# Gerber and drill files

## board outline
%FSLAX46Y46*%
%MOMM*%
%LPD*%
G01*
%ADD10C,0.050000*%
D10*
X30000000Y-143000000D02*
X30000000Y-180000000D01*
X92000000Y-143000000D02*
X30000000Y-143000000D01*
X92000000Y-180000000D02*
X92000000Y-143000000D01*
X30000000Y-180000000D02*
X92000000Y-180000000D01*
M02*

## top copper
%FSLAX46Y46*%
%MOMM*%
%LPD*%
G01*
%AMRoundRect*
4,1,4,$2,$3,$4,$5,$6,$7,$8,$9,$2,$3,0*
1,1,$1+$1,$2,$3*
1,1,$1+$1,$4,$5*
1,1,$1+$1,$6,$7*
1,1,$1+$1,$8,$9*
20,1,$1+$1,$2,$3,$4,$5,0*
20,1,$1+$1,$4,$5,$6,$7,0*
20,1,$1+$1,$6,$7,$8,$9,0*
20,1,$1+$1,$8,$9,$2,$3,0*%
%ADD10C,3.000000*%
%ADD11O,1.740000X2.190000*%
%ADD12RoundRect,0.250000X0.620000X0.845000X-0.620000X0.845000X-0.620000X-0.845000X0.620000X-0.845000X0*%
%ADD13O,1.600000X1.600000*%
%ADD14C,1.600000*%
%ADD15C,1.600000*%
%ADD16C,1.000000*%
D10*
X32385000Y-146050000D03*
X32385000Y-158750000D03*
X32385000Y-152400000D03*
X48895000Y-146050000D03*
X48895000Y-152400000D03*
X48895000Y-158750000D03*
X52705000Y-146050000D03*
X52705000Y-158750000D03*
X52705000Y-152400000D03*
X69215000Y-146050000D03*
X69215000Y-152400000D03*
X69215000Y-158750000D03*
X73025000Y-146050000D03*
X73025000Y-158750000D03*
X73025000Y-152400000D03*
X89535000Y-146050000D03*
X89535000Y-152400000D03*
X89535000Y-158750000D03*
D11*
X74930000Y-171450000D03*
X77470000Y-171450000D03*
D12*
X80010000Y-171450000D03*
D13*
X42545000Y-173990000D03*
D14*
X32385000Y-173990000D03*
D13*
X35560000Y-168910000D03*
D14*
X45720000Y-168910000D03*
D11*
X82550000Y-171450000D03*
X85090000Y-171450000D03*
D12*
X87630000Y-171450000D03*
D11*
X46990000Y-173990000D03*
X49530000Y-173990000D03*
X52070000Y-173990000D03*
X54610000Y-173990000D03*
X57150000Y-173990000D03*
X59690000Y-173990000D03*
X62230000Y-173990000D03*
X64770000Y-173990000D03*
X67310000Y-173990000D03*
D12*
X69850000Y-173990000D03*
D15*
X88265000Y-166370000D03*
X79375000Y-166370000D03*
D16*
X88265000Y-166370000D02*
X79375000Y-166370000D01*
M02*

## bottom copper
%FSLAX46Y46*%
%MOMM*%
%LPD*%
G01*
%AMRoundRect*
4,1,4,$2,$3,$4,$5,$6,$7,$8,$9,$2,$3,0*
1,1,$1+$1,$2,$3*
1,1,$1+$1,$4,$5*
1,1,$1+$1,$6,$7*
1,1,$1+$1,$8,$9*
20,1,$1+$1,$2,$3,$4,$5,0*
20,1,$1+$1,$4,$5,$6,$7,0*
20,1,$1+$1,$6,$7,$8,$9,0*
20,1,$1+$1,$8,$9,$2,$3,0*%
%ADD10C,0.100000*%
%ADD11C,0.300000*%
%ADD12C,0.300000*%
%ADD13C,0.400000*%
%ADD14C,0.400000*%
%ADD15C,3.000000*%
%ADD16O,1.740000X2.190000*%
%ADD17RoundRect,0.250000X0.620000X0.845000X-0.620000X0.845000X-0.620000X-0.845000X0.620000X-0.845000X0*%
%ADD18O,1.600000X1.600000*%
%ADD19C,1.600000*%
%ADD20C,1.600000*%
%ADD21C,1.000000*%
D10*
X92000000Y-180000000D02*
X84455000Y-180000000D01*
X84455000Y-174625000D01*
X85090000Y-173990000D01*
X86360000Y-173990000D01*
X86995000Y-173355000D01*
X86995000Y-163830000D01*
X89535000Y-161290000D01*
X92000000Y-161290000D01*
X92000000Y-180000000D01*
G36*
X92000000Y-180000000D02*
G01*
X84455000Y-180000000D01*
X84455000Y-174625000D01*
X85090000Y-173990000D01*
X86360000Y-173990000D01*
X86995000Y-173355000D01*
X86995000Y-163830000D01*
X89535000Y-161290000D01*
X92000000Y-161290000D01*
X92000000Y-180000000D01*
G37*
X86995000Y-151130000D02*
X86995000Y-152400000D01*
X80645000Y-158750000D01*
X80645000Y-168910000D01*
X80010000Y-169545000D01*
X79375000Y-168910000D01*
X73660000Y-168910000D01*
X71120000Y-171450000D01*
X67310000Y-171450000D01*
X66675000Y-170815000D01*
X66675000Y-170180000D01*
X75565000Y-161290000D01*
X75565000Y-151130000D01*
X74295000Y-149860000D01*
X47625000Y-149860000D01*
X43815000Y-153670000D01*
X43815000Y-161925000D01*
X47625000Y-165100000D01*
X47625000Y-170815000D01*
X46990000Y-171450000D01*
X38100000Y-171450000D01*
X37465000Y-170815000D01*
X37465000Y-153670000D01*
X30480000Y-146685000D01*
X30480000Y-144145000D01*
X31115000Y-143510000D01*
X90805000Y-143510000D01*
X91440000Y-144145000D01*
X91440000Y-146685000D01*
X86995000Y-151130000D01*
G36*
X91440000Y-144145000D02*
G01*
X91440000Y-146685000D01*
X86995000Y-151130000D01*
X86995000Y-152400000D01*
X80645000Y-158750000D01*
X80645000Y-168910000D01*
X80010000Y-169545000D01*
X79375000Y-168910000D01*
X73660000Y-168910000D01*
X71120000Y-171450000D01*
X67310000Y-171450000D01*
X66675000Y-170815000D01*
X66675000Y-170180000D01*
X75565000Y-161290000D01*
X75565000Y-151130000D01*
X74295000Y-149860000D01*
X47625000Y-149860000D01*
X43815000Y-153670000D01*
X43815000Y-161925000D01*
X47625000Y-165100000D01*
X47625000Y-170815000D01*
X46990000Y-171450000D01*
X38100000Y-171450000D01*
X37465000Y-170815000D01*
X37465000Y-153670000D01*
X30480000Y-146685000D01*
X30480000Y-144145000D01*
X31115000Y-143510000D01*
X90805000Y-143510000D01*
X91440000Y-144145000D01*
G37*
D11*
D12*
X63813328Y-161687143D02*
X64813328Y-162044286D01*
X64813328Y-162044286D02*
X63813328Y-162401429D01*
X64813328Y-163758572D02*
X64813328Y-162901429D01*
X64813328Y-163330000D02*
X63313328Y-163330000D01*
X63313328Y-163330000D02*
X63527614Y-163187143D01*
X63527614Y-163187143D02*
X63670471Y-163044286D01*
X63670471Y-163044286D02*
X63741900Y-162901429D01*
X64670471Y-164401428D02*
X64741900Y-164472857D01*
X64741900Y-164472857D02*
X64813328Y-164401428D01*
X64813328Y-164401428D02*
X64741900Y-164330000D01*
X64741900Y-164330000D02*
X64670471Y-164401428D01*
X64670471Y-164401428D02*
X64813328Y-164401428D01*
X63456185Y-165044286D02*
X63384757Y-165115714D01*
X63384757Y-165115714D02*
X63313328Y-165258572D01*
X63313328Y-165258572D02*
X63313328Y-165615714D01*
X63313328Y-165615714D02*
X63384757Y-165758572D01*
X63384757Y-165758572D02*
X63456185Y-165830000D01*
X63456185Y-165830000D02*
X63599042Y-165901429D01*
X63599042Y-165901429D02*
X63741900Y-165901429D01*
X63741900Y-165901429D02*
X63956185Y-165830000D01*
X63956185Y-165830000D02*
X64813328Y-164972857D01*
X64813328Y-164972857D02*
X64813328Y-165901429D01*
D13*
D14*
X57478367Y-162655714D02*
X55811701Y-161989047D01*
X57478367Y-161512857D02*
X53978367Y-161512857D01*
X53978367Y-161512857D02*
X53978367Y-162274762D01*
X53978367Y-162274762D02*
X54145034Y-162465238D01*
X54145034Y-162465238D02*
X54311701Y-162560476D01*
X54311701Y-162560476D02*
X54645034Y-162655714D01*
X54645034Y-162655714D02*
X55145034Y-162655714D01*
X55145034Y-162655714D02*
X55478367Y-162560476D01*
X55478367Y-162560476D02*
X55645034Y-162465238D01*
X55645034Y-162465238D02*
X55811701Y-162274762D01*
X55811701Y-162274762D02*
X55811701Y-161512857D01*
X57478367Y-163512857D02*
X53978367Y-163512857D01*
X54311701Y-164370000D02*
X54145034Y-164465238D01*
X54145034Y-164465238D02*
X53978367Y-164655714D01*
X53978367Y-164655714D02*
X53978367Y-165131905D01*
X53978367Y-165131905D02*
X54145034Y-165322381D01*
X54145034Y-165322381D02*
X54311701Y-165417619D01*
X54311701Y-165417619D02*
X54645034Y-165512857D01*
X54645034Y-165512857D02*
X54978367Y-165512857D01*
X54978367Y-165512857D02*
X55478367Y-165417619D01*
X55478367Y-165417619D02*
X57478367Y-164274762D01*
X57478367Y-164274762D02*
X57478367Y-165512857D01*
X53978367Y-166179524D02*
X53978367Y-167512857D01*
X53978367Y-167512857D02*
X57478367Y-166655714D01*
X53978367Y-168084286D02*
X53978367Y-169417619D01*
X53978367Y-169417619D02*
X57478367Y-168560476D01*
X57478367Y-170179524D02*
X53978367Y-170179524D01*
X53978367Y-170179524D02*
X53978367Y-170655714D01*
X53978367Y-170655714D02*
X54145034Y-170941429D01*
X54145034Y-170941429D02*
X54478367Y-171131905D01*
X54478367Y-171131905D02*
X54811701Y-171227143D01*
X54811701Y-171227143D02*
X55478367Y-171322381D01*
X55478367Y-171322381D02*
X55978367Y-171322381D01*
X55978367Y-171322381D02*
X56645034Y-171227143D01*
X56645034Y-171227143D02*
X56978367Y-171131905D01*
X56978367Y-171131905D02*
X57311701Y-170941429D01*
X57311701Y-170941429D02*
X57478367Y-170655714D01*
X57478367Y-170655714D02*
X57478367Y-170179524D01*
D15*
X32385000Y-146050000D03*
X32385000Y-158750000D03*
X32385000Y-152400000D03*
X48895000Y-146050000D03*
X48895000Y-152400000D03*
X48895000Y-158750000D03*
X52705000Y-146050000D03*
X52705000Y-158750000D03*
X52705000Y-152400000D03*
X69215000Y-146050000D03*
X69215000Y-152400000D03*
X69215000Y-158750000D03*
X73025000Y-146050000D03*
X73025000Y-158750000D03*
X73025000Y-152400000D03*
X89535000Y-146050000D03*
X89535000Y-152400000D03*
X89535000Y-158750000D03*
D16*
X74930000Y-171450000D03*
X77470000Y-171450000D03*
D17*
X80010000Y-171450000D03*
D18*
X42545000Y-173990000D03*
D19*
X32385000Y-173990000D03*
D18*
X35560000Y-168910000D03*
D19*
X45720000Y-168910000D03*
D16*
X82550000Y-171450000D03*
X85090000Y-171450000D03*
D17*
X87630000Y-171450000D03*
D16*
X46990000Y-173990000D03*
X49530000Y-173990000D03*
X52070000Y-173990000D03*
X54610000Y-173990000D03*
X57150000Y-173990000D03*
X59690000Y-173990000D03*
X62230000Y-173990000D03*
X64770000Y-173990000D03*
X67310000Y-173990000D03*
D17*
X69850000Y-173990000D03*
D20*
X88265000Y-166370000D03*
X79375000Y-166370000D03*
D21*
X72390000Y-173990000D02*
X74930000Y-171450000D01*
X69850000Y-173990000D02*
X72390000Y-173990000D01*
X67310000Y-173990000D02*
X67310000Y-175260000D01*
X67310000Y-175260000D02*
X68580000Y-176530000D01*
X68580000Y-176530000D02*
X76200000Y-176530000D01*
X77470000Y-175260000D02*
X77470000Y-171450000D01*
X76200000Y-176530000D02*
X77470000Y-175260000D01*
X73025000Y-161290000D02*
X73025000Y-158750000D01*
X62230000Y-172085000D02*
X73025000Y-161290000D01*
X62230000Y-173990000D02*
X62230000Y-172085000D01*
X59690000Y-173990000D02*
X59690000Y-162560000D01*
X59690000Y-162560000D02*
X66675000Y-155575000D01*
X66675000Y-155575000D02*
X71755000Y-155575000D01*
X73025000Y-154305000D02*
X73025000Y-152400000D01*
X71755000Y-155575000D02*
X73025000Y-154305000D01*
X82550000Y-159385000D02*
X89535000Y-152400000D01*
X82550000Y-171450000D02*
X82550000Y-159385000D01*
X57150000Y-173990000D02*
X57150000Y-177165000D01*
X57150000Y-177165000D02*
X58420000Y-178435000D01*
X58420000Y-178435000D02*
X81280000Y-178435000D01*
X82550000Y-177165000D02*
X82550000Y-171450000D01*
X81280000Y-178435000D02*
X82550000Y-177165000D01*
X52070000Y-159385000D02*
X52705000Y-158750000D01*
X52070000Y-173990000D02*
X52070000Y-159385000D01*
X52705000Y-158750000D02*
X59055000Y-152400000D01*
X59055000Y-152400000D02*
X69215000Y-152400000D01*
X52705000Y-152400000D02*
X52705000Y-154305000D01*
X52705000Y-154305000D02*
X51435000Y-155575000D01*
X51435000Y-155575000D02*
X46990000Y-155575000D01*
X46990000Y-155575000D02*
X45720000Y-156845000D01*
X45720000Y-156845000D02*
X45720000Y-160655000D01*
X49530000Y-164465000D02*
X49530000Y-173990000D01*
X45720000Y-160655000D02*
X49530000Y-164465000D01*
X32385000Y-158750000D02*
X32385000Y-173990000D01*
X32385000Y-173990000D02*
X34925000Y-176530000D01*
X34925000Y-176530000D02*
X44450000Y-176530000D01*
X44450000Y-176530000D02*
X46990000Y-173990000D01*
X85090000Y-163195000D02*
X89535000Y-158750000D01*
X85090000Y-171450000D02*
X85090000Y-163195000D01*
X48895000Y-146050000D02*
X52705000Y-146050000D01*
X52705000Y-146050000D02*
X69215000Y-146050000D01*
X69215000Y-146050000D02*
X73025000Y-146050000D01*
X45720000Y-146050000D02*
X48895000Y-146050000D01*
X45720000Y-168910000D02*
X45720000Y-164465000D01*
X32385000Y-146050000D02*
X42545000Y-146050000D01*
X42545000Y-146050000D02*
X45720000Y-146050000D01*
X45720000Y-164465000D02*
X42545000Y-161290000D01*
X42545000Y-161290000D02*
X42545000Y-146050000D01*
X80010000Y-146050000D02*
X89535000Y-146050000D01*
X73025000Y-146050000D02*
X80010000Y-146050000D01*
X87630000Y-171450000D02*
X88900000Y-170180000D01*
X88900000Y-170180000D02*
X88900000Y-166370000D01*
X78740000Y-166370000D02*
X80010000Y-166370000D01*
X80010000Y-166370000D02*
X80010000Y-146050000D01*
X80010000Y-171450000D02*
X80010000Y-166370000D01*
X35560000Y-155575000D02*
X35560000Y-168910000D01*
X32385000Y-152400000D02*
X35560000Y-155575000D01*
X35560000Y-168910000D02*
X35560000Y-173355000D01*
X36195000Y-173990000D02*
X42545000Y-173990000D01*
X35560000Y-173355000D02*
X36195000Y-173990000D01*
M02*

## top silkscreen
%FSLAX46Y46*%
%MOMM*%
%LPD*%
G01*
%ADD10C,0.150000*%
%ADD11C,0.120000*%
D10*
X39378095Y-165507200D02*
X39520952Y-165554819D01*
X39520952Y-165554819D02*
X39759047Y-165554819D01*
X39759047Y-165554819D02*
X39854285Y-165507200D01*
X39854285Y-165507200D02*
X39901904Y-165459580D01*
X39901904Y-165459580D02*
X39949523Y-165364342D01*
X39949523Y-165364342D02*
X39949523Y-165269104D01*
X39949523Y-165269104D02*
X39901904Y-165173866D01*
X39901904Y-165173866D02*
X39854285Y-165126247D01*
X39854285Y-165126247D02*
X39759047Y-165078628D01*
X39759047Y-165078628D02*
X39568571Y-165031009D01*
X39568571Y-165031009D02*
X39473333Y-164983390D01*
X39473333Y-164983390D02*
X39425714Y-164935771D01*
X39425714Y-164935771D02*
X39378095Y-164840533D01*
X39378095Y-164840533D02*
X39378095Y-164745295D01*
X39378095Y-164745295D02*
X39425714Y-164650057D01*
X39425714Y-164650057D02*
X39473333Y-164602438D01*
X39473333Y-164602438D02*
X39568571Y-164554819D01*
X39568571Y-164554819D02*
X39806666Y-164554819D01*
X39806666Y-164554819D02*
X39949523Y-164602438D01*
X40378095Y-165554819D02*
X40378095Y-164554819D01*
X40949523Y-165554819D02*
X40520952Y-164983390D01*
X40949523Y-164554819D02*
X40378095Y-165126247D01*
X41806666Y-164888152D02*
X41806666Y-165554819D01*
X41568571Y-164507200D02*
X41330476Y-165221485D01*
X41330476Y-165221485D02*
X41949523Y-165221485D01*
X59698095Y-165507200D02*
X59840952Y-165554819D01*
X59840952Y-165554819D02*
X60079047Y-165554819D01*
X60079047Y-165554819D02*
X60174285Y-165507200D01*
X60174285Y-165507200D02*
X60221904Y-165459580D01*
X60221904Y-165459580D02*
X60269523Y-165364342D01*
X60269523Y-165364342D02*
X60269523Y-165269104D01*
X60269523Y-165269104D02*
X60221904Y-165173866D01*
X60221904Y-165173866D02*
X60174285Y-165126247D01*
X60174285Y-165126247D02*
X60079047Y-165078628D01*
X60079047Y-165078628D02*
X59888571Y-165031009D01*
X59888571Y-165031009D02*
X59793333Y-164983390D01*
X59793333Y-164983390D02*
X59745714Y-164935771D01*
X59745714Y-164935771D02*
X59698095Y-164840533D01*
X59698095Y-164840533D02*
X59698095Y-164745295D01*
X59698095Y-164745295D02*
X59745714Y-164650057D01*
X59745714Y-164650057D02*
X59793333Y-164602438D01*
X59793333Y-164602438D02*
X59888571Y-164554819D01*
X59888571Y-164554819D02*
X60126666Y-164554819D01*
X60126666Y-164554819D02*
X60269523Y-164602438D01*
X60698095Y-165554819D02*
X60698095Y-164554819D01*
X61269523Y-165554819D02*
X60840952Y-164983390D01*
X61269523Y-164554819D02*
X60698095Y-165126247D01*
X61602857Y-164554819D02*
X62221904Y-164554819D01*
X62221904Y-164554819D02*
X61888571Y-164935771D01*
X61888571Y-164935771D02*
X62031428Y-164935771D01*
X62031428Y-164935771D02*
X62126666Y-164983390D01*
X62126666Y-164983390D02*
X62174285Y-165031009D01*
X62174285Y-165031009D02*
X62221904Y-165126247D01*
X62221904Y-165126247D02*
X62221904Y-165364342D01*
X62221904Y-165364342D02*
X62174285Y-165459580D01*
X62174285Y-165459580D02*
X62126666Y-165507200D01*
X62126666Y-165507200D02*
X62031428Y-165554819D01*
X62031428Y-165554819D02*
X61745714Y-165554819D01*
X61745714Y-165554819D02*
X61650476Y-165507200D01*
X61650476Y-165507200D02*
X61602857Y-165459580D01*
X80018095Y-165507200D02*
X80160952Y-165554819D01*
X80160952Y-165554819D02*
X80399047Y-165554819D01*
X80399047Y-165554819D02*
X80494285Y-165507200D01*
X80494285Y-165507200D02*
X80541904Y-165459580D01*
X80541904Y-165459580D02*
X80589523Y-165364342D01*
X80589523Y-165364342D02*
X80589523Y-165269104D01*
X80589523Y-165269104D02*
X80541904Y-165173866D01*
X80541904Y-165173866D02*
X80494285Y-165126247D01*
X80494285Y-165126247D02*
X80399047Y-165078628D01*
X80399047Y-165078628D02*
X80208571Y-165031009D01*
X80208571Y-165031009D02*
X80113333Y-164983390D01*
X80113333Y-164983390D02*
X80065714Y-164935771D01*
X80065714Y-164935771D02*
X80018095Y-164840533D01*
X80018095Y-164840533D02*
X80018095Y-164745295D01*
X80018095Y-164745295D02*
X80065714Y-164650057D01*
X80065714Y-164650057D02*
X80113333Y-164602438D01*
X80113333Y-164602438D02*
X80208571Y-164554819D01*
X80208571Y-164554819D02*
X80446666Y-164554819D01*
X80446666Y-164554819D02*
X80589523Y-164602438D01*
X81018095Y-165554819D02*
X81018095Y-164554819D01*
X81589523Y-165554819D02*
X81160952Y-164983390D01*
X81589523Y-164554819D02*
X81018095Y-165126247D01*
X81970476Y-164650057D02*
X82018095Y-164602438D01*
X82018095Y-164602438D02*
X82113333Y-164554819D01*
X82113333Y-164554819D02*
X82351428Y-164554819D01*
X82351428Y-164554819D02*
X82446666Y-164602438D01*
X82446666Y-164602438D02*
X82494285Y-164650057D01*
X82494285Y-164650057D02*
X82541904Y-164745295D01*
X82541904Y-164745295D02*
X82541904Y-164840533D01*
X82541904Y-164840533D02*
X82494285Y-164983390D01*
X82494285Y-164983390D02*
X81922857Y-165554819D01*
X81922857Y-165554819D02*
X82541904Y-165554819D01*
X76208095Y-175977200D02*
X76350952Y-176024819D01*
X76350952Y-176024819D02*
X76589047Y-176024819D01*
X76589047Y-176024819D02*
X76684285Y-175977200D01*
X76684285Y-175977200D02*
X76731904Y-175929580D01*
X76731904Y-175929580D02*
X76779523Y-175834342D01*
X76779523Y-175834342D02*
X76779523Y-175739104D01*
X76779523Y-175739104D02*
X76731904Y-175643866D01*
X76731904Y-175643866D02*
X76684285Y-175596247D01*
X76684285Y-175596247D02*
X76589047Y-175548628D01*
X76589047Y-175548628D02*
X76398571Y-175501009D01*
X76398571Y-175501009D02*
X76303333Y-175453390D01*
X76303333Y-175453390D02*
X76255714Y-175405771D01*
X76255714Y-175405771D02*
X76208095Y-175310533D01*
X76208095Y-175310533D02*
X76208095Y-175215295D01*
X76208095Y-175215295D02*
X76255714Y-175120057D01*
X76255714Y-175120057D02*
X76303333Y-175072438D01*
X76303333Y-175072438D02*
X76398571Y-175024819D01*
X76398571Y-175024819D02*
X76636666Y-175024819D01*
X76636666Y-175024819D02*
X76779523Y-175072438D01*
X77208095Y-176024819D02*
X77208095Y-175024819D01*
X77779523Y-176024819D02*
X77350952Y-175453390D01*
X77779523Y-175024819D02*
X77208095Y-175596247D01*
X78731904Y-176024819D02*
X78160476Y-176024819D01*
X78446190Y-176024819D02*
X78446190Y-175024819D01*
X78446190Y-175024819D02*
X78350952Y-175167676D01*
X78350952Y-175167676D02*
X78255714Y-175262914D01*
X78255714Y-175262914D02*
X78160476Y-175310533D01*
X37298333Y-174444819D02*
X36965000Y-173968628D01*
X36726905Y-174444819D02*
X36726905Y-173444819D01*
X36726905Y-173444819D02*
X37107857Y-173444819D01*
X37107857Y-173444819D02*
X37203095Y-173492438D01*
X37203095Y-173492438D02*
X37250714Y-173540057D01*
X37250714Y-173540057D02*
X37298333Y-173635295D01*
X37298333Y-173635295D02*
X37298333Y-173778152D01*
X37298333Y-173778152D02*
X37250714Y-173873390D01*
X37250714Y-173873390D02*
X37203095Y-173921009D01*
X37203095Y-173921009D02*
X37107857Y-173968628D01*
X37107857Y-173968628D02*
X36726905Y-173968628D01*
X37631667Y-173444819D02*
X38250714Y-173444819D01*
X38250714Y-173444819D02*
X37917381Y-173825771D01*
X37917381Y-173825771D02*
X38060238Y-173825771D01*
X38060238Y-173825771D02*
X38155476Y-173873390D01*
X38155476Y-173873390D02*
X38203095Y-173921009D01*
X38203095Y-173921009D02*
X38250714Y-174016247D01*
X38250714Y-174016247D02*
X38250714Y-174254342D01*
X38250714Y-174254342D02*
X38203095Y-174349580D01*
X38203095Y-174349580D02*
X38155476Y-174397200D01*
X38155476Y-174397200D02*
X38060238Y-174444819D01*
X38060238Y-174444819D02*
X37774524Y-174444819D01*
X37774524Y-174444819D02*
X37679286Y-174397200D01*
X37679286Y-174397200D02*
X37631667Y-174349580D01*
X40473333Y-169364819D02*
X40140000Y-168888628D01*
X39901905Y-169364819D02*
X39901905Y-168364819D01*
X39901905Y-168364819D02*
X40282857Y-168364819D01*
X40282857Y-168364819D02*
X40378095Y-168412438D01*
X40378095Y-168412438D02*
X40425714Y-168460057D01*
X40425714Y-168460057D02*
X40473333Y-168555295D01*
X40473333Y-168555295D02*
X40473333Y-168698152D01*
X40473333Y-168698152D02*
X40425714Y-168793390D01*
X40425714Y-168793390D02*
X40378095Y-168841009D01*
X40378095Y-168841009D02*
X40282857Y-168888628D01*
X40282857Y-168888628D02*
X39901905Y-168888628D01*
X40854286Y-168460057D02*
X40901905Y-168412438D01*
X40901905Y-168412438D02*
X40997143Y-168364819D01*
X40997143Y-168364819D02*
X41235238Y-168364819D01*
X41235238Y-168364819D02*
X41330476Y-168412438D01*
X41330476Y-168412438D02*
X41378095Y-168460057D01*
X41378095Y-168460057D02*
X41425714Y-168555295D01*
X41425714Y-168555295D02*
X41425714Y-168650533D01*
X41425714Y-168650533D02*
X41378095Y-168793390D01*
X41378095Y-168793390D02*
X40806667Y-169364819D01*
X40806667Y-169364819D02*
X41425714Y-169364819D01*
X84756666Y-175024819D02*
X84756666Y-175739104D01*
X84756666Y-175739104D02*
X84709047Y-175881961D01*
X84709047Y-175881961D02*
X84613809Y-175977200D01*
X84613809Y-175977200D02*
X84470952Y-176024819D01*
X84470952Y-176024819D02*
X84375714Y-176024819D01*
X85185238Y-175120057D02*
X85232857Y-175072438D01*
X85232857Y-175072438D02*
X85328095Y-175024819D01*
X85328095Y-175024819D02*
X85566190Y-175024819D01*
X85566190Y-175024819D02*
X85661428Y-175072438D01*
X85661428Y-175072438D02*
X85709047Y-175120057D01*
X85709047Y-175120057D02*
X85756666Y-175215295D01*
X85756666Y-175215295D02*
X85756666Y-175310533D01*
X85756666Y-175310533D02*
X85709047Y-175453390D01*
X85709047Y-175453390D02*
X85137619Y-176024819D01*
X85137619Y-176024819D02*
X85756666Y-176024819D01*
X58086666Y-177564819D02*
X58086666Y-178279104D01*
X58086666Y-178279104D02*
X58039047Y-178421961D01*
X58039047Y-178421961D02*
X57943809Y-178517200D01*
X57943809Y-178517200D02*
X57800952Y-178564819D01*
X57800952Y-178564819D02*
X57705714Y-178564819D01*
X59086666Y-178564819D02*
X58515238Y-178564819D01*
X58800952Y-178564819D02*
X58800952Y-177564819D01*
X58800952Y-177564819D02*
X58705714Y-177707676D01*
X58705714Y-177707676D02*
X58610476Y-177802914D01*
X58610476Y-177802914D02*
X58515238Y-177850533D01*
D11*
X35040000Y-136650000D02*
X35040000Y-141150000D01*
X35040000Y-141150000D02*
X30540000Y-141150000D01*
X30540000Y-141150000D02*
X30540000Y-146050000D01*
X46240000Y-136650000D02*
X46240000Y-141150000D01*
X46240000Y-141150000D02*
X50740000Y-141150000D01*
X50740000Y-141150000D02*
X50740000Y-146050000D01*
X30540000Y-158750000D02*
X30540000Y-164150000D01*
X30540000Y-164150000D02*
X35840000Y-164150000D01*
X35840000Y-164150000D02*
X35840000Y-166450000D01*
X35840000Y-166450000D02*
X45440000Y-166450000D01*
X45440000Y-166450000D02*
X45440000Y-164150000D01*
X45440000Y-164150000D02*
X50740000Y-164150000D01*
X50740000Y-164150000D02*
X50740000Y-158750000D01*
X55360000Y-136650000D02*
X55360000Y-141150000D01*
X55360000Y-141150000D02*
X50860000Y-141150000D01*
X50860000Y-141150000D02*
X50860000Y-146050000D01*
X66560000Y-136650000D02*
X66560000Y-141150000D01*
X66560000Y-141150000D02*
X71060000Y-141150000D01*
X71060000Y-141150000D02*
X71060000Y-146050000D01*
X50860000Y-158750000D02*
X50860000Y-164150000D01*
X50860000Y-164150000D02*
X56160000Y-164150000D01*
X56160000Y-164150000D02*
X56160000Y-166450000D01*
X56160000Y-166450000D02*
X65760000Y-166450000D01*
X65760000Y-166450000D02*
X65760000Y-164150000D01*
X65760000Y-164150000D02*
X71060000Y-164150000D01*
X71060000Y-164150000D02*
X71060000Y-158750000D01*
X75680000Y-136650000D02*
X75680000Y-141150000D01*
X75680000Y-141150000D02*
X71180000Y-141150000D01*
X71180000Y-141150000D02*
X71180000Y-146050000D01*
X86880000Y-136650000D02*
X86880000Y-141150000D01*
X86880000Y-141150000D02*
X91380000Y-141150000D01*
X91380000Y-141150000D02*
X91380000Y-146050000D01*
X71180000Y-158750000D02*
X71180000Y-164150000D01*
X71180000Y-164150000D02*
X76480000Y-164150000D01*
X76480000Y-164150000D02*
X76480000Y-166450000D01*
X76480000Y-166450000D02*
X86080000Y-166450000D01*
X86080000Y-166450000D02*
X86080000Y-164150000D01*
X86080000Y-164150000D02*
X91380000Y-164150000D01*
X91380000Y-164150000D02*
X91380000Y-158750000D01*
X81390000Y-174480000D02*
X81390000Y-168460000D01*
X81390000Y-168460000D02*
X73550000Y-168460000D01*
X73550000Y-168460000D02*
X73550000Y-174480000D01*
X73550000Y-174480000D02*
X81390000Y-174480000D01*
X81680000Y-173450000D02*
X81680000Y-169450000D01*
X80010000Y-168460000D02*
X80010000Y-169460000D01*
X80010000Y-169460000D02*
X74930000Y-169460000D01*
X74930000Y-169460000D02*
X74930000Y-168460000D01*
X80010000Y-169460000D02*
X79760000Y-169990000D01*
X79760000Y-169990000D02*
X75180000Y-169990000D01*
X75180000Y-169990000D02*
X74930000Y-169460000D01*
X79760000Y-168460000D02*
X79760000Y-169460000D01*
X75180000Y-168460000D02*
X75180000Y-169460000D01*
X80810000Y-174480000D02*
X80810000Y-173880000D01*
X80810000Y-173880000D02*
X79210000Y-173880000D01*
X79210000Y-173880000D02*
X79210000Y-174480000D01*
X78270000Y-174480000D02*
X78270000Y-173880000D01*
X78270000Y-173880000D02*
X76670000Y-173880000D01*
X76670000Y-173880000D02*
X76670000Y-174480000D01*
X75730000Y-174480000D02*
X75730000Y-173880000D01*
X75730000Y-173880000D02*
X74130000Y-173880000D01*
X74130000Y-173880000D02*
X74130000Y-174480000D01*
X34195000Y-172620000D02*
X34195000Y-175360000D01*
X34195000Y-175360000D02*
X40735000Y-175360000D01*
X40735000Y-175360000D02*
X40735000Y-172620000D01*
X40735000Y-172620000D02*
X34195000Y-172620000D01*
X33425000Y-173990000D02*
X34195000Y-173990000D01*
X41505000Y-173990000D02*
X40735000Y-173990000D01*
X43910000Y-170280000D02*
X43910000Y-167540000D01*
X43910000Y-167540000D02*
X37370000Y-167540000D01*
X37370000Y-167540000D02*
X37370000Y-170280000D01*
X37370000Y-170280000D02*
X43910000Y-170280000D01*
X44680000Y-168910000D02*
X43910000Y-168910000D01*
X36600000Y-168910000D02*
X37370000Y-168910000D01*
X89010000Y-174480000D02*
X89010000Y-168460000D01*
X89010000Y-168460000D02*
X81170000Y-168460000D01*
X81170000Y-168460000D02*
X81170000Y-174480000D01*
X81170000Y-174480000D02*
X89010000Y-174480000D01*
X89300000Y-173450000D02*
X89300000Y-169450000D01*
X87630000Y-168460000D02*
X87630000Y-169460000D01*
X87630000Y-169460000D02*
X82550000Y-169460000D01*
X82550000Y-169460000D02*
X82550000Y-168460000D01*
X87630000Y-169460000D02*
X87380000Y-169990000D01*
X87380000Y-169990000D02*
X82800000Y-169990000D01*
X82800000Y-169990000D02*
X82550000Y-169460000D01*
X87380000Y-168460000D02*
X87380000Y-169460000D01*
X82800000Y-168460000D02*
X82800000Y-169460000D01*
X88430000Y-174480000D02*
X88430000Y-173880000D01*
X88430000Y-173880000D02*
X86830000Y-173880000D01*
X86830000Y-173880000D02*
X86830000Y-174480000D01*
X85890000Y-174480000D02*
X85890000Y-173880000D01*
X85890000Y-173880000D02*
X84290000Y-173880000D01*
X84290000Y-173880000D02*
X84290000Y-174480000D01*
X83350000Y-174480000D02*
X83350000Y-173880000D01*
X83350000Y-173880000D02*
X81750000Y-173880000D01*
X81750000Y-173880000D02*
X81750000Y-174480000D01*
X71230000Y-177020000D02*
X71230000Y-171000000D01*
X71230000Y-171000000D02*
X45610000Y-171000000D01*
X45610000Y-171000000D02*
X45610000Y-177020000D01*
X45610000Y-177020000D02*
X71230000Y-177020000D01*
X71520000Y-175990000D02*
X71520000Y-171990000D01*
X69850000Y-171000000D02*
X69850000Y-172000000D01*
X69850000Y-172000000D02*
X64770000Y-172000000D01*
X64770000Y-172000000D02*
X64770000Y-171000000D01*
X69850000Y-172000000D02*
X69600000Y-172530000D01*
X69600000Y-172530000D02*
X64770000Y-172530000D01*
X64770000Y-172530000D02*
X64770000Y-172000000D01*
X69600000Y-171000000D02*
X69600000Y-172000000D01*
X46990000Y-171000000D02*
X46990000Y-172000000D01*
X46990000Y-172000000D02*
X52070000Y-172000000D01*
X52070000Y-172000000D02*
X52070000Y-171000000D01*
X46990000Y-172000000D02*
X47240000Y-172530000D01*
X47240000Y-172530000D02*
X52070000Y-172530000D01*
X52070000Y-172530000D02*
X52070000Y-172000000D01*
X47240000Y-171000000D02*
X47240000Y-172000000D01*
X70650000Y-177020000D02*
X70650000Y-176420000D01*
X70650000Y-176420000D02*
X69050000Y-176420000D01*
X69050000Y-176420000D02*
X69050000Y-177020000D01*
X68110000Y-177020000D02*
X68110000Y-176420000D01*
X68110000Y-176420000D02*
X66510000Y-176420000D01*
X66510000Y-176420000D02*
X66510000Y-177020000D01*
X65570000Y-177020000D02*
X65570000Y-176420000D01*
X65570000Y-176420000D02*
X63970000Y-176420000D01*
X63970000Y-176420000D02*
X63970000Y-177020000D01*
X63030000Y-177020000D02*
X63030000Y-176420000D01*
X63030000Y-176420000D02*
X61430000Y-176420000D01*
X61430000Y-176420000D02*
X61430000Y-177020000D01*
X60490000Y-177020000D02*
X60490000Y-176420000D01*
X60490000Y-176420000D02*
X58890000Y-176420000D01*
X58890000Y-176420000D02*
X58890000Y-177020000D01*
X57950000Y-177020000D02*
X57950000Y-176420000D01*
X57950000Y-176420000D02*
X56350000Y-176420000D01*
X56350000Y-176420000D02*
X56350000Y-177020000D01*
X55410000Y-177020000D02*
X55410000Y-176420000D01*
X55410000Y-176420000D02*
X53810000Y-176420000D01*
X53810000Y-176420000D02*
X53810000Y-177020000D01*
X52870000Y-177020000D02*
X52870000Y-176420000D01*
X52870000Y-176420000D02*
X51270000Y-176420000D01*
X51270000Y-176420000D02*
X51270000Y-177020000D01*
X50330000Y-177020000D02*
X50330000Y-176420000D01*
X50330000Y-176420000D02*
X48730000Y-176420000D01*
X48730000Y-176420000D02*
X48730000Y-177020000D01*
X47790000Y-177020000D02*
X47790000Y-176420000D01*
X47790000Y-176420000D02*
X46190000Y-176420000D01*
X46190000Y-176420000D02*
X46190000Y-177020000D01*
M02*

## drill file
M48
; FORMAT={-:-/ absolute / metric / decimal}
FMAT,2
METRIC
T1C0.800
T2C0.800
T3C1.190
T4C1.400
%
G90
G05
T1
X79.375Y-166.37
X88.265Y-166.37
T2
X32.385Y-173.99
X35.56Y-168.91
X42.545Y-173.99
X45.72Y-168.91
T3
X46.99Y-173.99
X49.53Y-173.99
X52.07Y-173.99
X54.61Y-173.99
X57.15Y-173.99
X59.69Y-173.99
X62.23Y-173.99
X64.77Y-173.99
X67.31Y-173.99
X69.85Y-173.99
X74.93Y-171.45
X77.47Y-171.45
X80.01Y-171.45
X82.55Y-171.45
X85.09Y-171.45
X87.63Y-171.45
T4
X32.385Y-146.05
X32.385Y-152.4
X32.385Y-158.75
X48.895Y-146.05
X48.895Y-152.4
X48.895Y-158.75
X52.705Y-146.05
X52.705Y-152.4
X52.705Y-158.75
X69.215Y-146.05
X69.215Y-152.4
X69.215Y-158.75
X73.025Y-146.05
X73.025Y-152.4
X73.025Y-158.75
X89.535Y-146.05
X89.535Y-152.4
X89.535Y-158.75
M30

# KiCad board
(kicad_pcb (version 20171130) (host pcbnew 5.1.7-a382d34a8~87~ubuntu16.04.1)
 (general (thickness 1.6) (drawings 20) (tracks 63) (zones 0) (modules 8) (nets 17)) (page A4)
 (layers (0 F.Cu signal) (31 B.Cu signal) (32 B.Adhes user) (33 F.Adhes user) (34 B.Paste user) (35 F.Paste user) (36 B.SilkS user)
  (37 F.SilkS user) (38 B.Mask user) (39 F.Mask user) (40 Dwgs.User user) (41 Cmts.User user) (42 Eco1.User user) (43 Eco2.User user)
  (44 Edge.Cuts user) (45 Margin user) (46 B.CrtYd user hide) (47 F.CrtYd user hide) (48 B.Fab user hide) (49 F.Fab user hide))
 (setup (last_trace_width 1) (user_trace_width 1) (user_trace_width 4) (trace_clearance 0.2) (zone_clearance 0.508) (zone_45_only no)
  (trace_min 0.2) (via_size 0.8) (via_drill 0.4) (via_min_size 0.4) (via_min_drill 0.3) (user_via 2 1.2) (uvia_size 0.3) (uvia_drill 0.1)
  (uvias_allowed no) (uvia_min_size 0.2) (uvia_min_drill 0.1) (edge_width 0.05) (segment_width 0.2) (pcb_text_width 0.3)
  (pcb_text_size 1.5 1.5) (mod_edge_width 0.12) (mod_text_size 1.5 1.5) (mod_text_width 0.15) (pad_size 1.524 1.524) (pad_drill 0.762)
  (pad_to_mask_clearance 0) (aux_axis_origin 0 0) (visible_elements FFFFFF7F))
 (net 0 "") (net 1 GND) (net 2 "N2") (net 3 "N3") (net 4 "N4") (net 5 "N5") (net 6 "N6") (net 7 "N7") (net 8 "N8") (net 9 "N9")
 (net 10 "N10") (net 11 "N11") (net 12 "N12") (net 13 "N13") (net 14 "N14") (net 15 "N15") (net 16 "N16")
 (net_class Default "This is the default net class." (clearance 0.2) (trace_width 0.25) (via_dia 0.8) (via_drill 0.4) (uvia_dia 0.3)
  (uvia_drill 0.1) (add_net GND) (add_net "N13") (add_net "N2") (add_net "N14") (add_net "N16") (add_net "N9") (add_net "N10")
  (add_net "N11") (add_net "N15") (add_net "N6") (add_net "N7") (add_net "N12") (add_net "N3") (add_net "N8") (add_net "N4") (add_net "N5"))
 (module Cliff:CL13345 (layer F.Cu) (at 40.64 146.05 90)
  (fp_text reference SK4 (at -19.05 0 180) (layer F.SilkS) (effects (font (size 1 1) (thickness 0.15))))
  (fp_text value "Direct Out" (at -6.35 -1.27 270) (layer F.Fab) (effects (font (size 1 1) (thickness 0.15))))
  (fp_line (start 9.4 -5.6) (end 4.9 -5.6) (layer F.SilkS) (width 0.12))
  (fp_line (start 4.9 -5.6) (end 4.9 -10.1) (layer F.SilkS) (width 0.12))
  (fp_line (start 4.9 -10.1) (end 0 -10.1) (layer F.SilkS) (width 0.12))
  (fp_line (start 9.4 5.6) (end 4.9 5.6) (layer F.SilkS) (width 0.12))
  (fp_line (start 4.9 5.6) (end 4.9 10.1) (layer F.SilkS) (width 0.12))
  (fp_line (start 4.9 10.1) (end 0 10.1) (layer F.SilkS) (width 0.12))
  (fp_line (start -12.7 -10.1) (end -18.1 -10.1) (layer F.SilkS) (width 0.12))
  (fp_line (start -18.1 -10.1) (end -18.1 -4.8) (layer F.SilkS) (width 0.12))
  (fp_line (start -18.1 -4.8) (end -20.4 -4.8) (layer F.SilkS) (width 0.12))
  (fp_line (start -20.4 -4.8) (end -20.4 4.8) (layer F.SilkS) (width 0.12))
  (fp_line (start -20.4 4.8) (end -18.1 4.8) (layer F.SilkS) (width 0.12))
  (fp_line (start -18.1 4.8) (end -18.1 10.1) (layer F.SilkS) (width 0.12))
  (fp_line (start -18.1 10.1) (end -12.7 10.1) (layer F.SilkS) (width 0.12))
  (pad S thru_hole circle (at 0 -8.255 180) (size 3 3) (drill 1.4) (layers *.Cu *.Mask) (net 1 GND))
  (pad T thru_hole circle (at -12.7 -8.255 180) (size 3 3) (drill 1.4) (layers *.Cu *.Mask) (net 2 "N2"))
  (pad R thru_hole circle (at -6.35 -8.255 180) (size 3 3) (drill 1.4) (layers *.Cu *.Mask) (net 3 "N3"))
  (pad SN thru_hole circle (at 0 8.255 180) (size 3 3) (drill 1.4) (layers *.Cu *.Mask) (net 1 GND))
  (pad RN thru_hole circle (at -6.35 8.255 180) (size 3 3) (drill 1.4) (layers *.Cu *.Mask) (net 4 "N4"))
  (pad TN thru_hole circle (at -12.7 8.255 180) (size 3 3) (drill 1.4) (layers *.Cu *.Mask) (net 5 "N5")))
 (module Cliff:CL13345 (layer F.Cu) (at 60.96 146.05 90)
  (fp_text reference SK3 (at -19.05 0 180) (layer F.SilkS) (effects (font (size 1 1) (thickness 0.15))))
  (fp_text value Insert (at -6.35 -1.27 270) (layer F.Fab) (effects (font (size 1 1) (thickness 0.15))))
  (fp_line (start 9.4 -5.6) (end 4.9 -5.6) (layer F.SilkS) (width 0.12))
  (fp_line (start 4.9 -5.6) (end 4.9 -10.1) (layer F.SilkS) (width 0.12))
  (fp_line (start 4.9 -10.1) (end 0 -10.1) (layer F.SilkS) (width 0.12))
  (fp_line (start 9.4 5.6) (end 4.9 5.6) (layer F.SilkS) (width 0.12))
  (fp_line (start 4.9 5.6) (end 4.9 10.1) (layer F.SilkS) (width 0.12))
  (fp_line (start 4.9 10.1) (end 0 10.1) (layer F.SilkS) (width 0.12))
  (fp_line (start -12.7 -10.1) (end -18.1 -10.1) (layer F.SilkS) (width 0.12))
  (fp_line (start -18.1 -10.1) (end -18.1 -4.8) (layer F.SilkS) (width 0.12))
  (fp_line (start -18.1 -4.8) (end -20.4 -4.8) (layer F.SilkS) (width 0.12))
  (fp_line (start -20.4 -4.8) (end -20.4 4.8) (layer F.SilkS) (width 0.12))
  (fp_line (start -20.4 4.8) (end -18.1 4.8) (layer F.SilkS) (width 0.12))
  (fp_line (start -18.1 4.8) (end -18.1 10.1) (layer F.SilkS) (width 0.12))
  (fp_line (start -18.1 10.1) (end -12.7 10.1) (layer F.SilkS) (width 0.12))
  (pad S thru_hole circle (at 0 -8.255 180) (size 3 3) (drill 1.4) (layers *.Cu *.Mask) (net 1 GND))
  (pad T thru_hole circle (at -12.7 -8.255 180) (size 3 3) (drill 1.4) (layers *.Cu *.Mask) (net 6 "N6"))
  (pad R thru_hole circle (at -6.35 -8.255 180) (size 3 3) (drill 1.4) (layers *.Cu *.Mask) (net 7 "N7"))
  (pad SN thru_hole circle (at 0 8.255 180) (size 3 3) (drill 1.4) (layers *.Cu *.Mask) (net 1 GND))
  (pad RN thru_hole circle (at -6.35 8.255 180) (size 3 3) (drill 1.4) (layers *.Cu *.Mask) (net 6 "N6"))
  (pad TN thru_hole circle (at -12.7 8.255 180) (size 3 3) (drill 1.4) (layers *.Cu *.Mask) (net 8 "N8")))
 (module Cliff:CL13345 (layer F.Cu) (at 81.28 146.05 90)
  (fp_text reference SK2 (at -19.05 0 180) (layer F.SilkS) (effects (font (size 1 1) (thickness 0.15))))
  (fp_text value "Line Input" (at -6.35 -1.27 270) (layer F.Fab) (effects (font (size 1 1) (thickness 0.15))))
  (fp_line (start 9.4 -5.6) (end 4.9 -5.6) (layer F.SilkS) (width 0.12))
  (fp_line (start 4.9 -5.6) (end 4.9 -10.1) (layer F.SilkS) (width 0.12))
  (fp_line (start 4.9 -10.1) (end 0 -10.1) (layer F.SilkS) (width 0.12))
  (fp_line (start 9.4 5.6) (end 4.9 5.6) (layer F.SilkS) (width 0.12))
  (fp_line (start 4.9 5.6) (end 4.9 10.1) (layer F.SilkS) (width 0.12))
  (fp_line (start 4.9 10.1) (end 0 10.1) (layer F.SilkS) (width 0.12))
  (fp_line (start -12.7 -10.1) (end -18.1 -10.1) (layer F.SilkS) (width 0.12))
  (fp_line (start -18.1 -10.1) (end -18.1 -4.8) (layer F.SilkS) (width 0.12))
  (fp_line (start -18.1 -4.8) (end -20.4 -4.8) (layer F.SilkS) (width 0.12))
  (fp_line (start -20.4 -4.8) (end -20.4 4.8) (layer F.SilkS) (width 0.12))
  (fp_line (start -20.4 4.8) (end -18.1 4.8) (layer F.SilkS) (width 0.12))
  (fp_line (start -18.1 4.8) (end -18.1 10.1) (layer F.SilkS) (width 0.12))
  (fp_line (start -18.1 10.1) (end -12.7 10.1) (layer F.SilkS) (width 0.12))
  (pad S thru_hole circle (at 0 -8.255 180) (size 3 3) (drill 1.4) (layers *.Cu *.Mask) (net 1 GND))
  (pad T thru_hole circle (at -12.7 -8.255 180) (size 3 3) (drill 1.4) (layers *.Cu *.Mask) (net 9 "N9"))
  (pad R thru_hole circle (at -6.35 -8.255 180) (size 3 3) (drill 1.4) (layers *.Cu *.Mask) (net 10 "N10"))
  (pad SN thru_hole circle (at 0 8.255 180) (size 3 3) (drill 1.4) (layers *.Cu *.Mask) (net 1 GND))
  (pad RN thru_hole circle (at -6.35 8.255 180) (size 3 3) (drill 1.4) (layers *.Cu *.Mask) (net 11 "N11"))
  (pad TN thru_hole circle (at -12.7 8.255 180) (size 3 3) (drill 1.4) (layers *.Cu *.Mask) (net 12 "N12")))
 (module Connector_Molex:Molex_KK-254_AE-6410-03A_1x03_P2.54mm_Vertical (layer F.Cu) (at 80.01 171.45 180)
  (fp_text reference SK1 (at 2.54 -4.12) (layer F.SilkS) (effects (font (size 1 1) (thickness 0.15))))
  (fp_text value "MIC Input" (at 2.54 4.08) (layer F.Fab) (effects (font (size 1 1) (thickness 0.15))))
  (fp_line (start -1.38 -3.03) (end -1.38 2.99) (layer F.SilkS) (width 0.12))
  (fp_line (start -1.38 2.99) (end 6.46 2.99) (layer F.SilkS) (width 0.12))
  (fp_line (start 6.46 2.99) (end 6.46 -3.03) (layer F.SilkS) (width 0.12))
  (fp_line (start 6.46 -3.03) (end -1.38 -3.03) (layer F.SilkS) (width 0.12))
  (fp_line (start -1.67 -2) (end -1.67 2) (layer F.SilkS) (width 0.12))
  (fp_line (start 0 2.99) (end 0 1.99) (layer F.SilkS) (width 0.12))
  (fp_line (start 0 1.99) (end 5.08 1.99) (layer F.SilkS) (width 0.12))
  (fp_line (start 5.08 1.99) (end 5.08 2.99) (layer F.SilkS) (width 0.12))
  (fp_line (start 0 1.99) (end 0.25 1.46) (layer F.SilkS) (width 0.12))
  (fp_line (start 0.25 1.46) (end 4.83 1.46) (layer F.SilkS) (width 0.12))
  (fp_line (start 4.83 1.46) (end 5.08 1.99) (layer F.SilkS) (width 0.12))
  (fp_line (start 0.25 2.99) (end 0.25 1.99) (layer F.SilkS) (width 0.12))
  (fp_line (start 4.83 2.99) (end 4.83 1.99) (layer F.SilkS) (width 0.12))
  (fp_line (start -0.8 -3.03) (end -0.8 -2.43) (layer F.SilkS) (width 0.12))
  (fp_line (start -0.8 -2.43) (end 0.8 -2.43) (layer F.SilkS) (width 0.12))
  (fp_line (start 0.8 -2.43) (end 0.8 -3.03) (layer F.SilkS) (width 0.12))
  (fp_line (start 1.74 -3.03) (end 1.74 -2.43) (layer F.SilkS) (width 0.12))
  (fp_line (start 1.74 -2.43) (end 3.34 -2.43) (layer F.SilkS) (width 0.12))
  (fp_line (start 3.34 -2.43) (end 3.34 -3.03) (layer F.SilkS) (width 0.12))
  (fp_line (start 4.28 -3.03) (end 4.28 -2.43) (layer F.SilkS) (width 0.12))
  (fp_line (start 4.28 -2.43) (end 5.88 -2.43) (layer F.SilkS) (width 0.12))
  (fp_line (start 5.88 -2.43) (end 5.88 -3.03) (layer F.SilkS) (width 0.12))
  (pad 3 thru_hole oval (at 5.08 0 180) (size 1.74 2.19) (drill 1.19) (layers *.Cu *.Mask) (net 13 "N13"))
  (pad 2 thru_hole oval (at 2.54 0 180) (size 1.74 2.19) (drill 1.19) (layers *.Cu *.Mask) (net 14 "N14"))
  (pad 1 thru_hole roundrect (at 0 0 180) (size 1.74 2.19) (drill 1.19) (layers *.Cu *.Mask) (roundrect_rratio 0.143678) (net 1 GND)))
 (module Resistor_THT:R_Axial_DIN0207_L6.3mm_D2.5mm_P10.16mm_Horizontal (layer F.Cu) (at 32.385 173.99)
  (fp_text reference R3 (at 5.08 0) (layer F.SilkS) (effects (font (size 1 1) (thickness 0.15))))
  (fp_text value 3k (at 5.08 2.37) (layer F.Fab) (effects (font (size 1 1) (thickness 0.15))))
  (fp_line (start 1.81 -1.37) (end 1.81 1.37) (layer F.SilkS) (width 0.12))
  (fp_line (start 1.81 1.37) (end 8.35 1.37) (layer F.SilkS) (width 0.12))
  (fp_line (start 8.35 1.37) (end 8.35 -1.37) (layer F.SilkS) (width 0.12))
  (fp_line (start 8.35 -1.37) (end 1.81 -1.37) (layer F.SilkS) (width 0.12))
  (fp_line (start 1.04 0) (end 1.81 0) (layer F.SilkS) (width 0.12))
  (fp_line (start 9.12 0) (end 8.35 0) (layer F.SilkS) (width 0.12))
  (pad 2 thru_hole oval (at 10.16 0) (size 1.6 1.6) (drill 0.8) (layers *.Cu *.Mask) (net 3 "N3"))
  (pad 1 thru_hole circle (at 0 0) (size 1.6 1.6) (drill 0.8) (layers *.Cu *.Mask) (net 2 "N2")))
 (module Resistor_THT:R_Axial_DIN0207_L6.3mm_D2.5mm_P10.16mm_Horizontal (layer F.Cu) (at 45.72 168.91 180)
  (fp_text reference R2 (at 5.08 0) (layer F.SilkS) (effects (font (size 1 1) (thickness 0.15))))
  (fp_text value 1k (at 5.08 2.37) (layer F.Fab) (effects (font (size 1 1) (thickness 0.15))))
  (fp_line (start 1.81 -1.37) (end 1.81 1.37) (layer F.SilkS) (width 0.12))
  (fp_line (start 1.81 1.37) (end 8.35 1.37) (layer F.SilkS) (width 0.12))
  (fp_line (start 8.35 1.37) (end 8.35 -1.37) (layer F.SilkS) (width 0.12))
  (fp_line (start 8.35 -1.37) (end 1.81 -1.37) (layer F.SilkS) (width 0.12))
  (fp_line (start 1.04 0) (end 1.81 0) (layer F.SilkS) (width 0.12))
  (fp_line (start 9.12 0) (end 8.35 0) (layer F.SilkS) (width 0.12))
  (pad 2 thru_hole oval (at 10.16 0 180) (size 1.6 1.6) (drill 0.8) (layers *.Cu *.Mask) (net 3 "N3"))
  (pad 1 thru_hole circle (at 0 0 180) (size 1.6 1.6) (drill 0.8) (layers *.Cu *.Mask) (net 1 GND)))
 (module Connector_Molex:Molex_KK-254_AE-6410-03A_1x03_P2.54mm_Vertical (layer F.Cu) (at 87.63 171.45 180)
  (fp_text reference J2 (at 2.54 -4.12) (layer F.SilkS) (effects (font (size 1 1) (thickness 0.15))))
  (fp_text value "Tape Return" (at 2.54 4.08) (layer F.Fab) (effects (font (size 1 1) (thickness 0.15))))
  (fp_line (start -1.38 -3.03) (end -1.38 2.99) (layer F.SilkS) (width 0.12))
  (fp_line (start -1.38 2.99) (end 6.46 2.99) (layer F.SilkS) (width 0.12))
  (fp_line (start 6.46 2.99) (end 6.46 -3.03) (layer F.SilkS) (width 0.12))
  (fp_line (start 6.46 -3.03) (end -1.38 -3.03) (layer F.SilkS) (width 0.12))
  (fp_line (start -1.67 -2) (end -1.67 2) (layer F.SilkS) (width 0.12))
  (fp_line (start 0 2.99) (end 0 1.99) (layer F.SilkS) (width 0.12))
  (fp_line (start 0 1.99) (end 5.08 1.99) (layer F.SilkS) (width 0.12))
  (fp_line (start 5.08 1.99) (end 5.08 2.99) (layer F.SilkS) (width 0.12))
  (fp_line (start 0 1.99) (end 0.25 1.46) (layer F.SilkS) (width 0.12))
  (fp_line (start 0.25 1.46) (end 4.83 1.46) (layer F.SilkS) (width 0.12))
  (fp_line (start 4.83 1.46) (end 5.08 1.99) (layer F.SilkS) (width 0.12))
  (fp_line (start 0.25 2.99) (end 0.25 1.99) (layer F.SilkS) (width 0.12))
  (fp_line (start 4.83 2.99) (end 4.83 1.99) (layer F.SilkS) (width 0.12))
  (fp_line (start -0.8 -3.03) (end -0.8 -2.43) (layer F.SilkS) (width 0.12))
  (fp_line (start -0.8 -2.43) (end 0.8 -2.43) (layer F.SilkS) (width 0.12))
  (fp_line (start 0.8 -2.43) (end 0.8 -3.03) (layer F.SilkS) (width 0.12))
  (fp_line (start 1.74 -3.03) (end 1.74 -2.43) (layer F.SilkS) (width 0.12))
  (fp_line (start 1.74 -2.43) (end 3.34 -2.43) (layer F.SilkS) (width 0.12))
  (fp_line (start 3.34 -2.43) (end 3.34 -3.03) (layer F.SilkS) (width 0.12))
  (fp_line (start 4.28 -3.03) (end 4.28 -2.43) (layer F.SilkS) (width 0.12))
  (fp_line (start 4.28 -2.43) (end 5.88 -2.43) (layer F.SilkS) (width 0.12))
  (fp_line (start 5.88 -2.43) (end 5.88 -3.03) (layer F.SilkS) (width 0.12))
  (pad 3 thru_hole oval (at 5.08 0 180) (size 1.74 2.19) (drill 1.19) (layers *.Cu *.Mask) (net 11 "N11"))
  (pad 2 thru_hole oval (at 2.54 0 180) (size 1.74 2.19) (drill 1.19) (layers *.Cu *.Mask) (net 12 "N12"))
  (pad 1 thru_hole roundrect (at 0 0 180) (size 1.74 2.19) (drill 1.19) (layers *.Cu *.Mask) (roundrect_rratio 0.143678) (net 1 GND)))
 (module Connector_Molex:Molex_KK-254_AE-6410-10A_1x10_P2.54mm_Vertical (layer F.Cu) (at 69.85 173.99 180)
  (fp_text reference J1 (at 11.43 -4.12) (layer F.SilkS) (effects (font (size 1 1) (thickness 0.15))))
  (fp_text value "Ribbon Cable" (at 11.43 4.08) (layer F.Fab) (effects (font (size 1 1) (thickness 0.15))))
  (fp_line (start -1.38 -3.03) (end -1.38 2.99) (layer F.SilkS) (width 0.12))
  (fp_line (start -1.38 2.99) (end 24.24 2.99) (layer F.SilkS) (width 0.12))
  (fp_line (start 24.24 2.99) (end 24.24 -3.03) (layer F.SilkS) (width 0.12))
  (fp_line (start 24.24 -3.03) (end -1.38 -3.03) (layer F.SilkS) (width 0.12))
  (fp_line (start -1.67 -2) (end -1.67 2) (layer F.SilkS) (width 0.12))
  (fp_line (start 0 2.99) (end 0 1.99) (layer F.SilkS) (width 0.12))
  (fp_line (start 0 1.99) (end 5.08 1.99) (layer F.SilkS) (width 0.12))
  (fp_line (start 5.08 1.99) (end 5.08 2.99) (layer F.SilkS) (width 0.12))
  (fp_line (start 0 1.99) (end 0.25 1.46) (layer F.SilkS) (width 0.12))
  (fp_line (start 0.25 1.46) (end 5.08 1.46) (layer F.SilkS) (width 0.12))
  (fp_line (start 5.08 1.46) (end 5.08 1.99) (layer F.SilkS) (width 0.12))
  (fp_line (start 0.25 2.99) (end 0.25 1.99) (layer F.SilkS) (width 0.12))
  (fp_line (start 22.86 2.99) (end 22.86 1.99) (layer F.SilkS) (width 0.12))
  (fp_line (start 22.86 1.99) (end 17.78 1.99) (layer F.SilkS) (width 0.12))
  (fp_line (start 17.78 1.99) (end 17.78 2.99) (layer F.SilkS) (width 0.12))
  (fp_line (start 22.86 1.99) (end 22.61 1.46) (layer F.SilkS) (width 0.12))
  (fp_line (start 22.61 1.46) (end 17.78 1.46) (layer F.SilkS) (width 0.12))
  (fp_line (start 17.78 1.46) (end 17.78 1.99) (layer F.SilkS) (width 0.12))
  (fp_line (start 22.61 2.99) (end 22.61 1.99) (layer F.SilkS) (width 0.12))
  (fp_line (start -0.8 -3.03) (end -0.8 -2.43) (layer F.SilkS) (width 0.12))
  (fp_line (start -0.8 -2.43) (end 0.8 -2.43) (layer F.SilkS) (width 0.12))
  (fp_line (start 0.8 -2.43) (end 0.8 -3.03) (layer F.SilkS) (width 0.12))
  (fp_line (start 1.74 -3.03) (end 1.74 -2.43) (layer F.SilkS) (width 0.12))
  (fp_line (start 1.74 -2.43) (end 3.34 -2.43) (layer F.SilkS) (width 0.12))
  (fp_line (start 3.34 -2.43) (end 3.34 -3.03) (layer F.SilkS) (width 0.12))
  (fp_line (start 4.28 -3.03) (end 4.28 -2.43) (layer F.SilkS) (width 0.12))
  (fp_line (start 4.28 -2.43) (end 5.88 -2.43) (layer F.SilkS) (width 0.12))
  (fp_line (start 5.88 -2.43) (end 5.88 -3.03) (layer F.SilkS) (width 0.12))
  (fp_line (start 6.82 -3.03) (end 6.82 -2.43) (layer F.SilkS) (width 0.12))
  (fp_line (start 6.82 -2.43) (end 8.42 -2.43) (layer F.SilkS) (width 0.12))
  (fp_line (start 8.42 -2.43) (end 8.42 -3.03) (layer F.SilkS) (width 0.12))
  (fp_line (start 9.36 -3.03) (end 9.36 -2.43) (layer F.SilkS) (width 0.12))
  (fp_line (start 9.36 -2.43) (end 10.96 -2.43) (layer F.SilkS) (width 0.12))
  (fp_line (start 10.96 -2.43) (end 10.96 -3.03) (layer F.SilkS) (width 0.12))
  (fp_line (start 11.9 -3.03) (end 11.9 -2.43) (layer F.SilkS) (width 0.12))
  (fp_line (start 11.9 -2.43) (end 13.5 -2.43) (layer F.SilkS) (width 0.12))
  (fp_line (start 13.5 -2.43) (end 13.5 -3.03) (layer F.SilkS) (width 0.12))
  (fp_line (start 14.44 -3.03) (end 14.44 -2.43) (layer F.SilkS) (width 0.12))
  (fp_line (start 14.44 -2.43) (end 16.04 -2.43) (layer F.SilkS) (width 0.12))
  (fp_line (start 16.04 -2.43) (end 16.04 -3.03) (layer F.SilkS) (width 0.12))
  (fp_line (start 16.98 -3.03) (end 16.98 -2.43) (layer F.SilkS) (width 0.12))
  (fp_line (start 16.98 -2.43) (end 18.58 -2.43) (layer F.SilkS) (width 0.12))
  (fp_line (start 18.58 -2.43) (end 18.58 -3.03) (layer F.SilkS) (width 0.12))
  (fp_line (start 19.52 -3.03) (end 19.52 -2.43) (layer F.SilkS) (width 0.12))
  (fp_line (start 19.52 -2.43) (end 21.12 -2.43) (layer F.SilkS) (width 0.12))
  (fp_line (start 21.12 -2.43) (end 21.12 -3.03) (layer F.SilkS) (width 0.12))
  (fp_line (start 22.06 -3.03) (end 22.06 -2.43) (layer F.SilkS) (width 0.12))
  (fp_line (start 22.06 -2.43) (end 23.66 -2.43) (layer F.SilkS) (width 0.12))
  (fp_line (start 23.66 -2.43) (end 23.66 -3.03) (layer F.SilkS) (width 0.12))
  (pad 10 thru_hole oval (at 22.86 0 180) (size 1.74 2.19) (drill 1.19) (layers *.Cu *.Mask) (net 2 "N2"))
  (pad 9 thru_hole oval (at 20.32 0 180) (size 1.74 2.19) (drill 1.19) (layers *.Cu *.Mask) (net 7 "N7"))
  (pad 8 thru_hole oval (at 17.78 0 180) (size 1.74 2.19) (drill 1.19) (layers *.Cu *.Mask) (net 6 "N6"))
  (pad 7 thru_hole oval (at 15.24 0 180) (size 1.74 2.19) (drill 1.19) (layers *.Cu *.Mask) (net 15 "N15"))
  (pad 6 thru_hole oval (at 12.7 0 180) (size 1.74 2.19) (drill 1.19) (layers *.Cu *.Mask) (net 11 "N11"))
  (pad 5 thru_hole oval (at 10.16 0 180) (size 1.74 2.19) (drill 1.19) (layers *.Cu *.Mask) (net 10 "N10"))
  (pad 4 thru_hole oval (at 7.62 0 180) (size 1.74 2.19) (drill 1.19) (layers *.Cu *.Mask) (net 9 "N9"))
  (pad 3 thru_hole oval (at 5.08 0 180) (size 1.74 2.19) (drill 1.19) (layers *.Cu *.Mask) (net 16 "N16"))
  (pad 2 thru_hole oval (at 2.54 0 180) (size 1.74 2.19) (drill 1.19) (layers *.Cu *.Mask) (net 14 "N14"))
  (pad 1 thru_hole roundrect (at 0 0 180) (size 1.74 2.19) (drill 1.19) (layers *.Cu *.Mask) (roundrect_rratio 0.143678) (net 13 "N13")))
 (gr_poly
  (pts (xy 92 180) (xy 84.455 180) (xy 84.455 174.625) (xy 85.09 173.99) (xy 86.36 173.99) (xy 86.995 173.355) (xy 86.995 163.83)
   (xy 89.535 161.29) (xy 92 161.29))
  (layer B.Cu) (width 0.1))
 (gr_poly
  (pts (xy 86.995 151.13) (xy 86.995 152.4) (xy 80.645 158.75) (xy 80.645 168.91) (xy 80.01 169.545) (xy 79.375 168.91) (xy 73.66 168.91)
   (xy 71.12 171.45) (xy 67.31 171.45) (xy 66.675 170.815) (xy 66.675 170.18) (xy 75.565 161.29) (xy 75.565 151.13) (xy 74.295 149.86)
   (xy 47.625 149.86) (xy 43.815 153.67) (xy 43.815 161.925) (xy 47.625 165.1) (xy 47.625 170.815) (xy 46.99 171.45) (xy 38.1 171.45)
   (xy 37.465 170.815) (xy 37.465 153.67) (xy 30.48 146.685) (xy 30.48 144.145) (xy 31.115 143.51) (xy 90.805 143.51) (xy 91.44 144.145)
   (xy 91.44 146.685))
  (layer B.Cu) (width 0.1))
 (gr_line (start 30 143) (end 30 180) (layer Edge.Cuts) (width 0.05))
 (gr_line (start 92 143) (end 30 143) (layer Edge.Cuts) (width 0.05))
 (gr_line (start 92 180) (end 92 143) (layer Edge.Cuts) (width 0.05))
 (gr_line (start 30 180) (end 92 180) (layer Edge.Cuts) (width 0.05))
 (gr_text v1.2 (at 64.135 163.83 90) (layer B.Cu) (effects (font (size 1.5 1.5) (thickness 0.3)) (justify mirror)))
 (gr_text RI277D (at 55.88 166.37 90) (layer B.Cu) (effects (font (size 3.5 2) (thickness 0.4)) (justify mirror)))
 (segment (start 72.39 173.99) (end 74.93 171.45) (width 1) (layer B.Cu) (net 13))
 (segment (start 69.85 173.99) (end 72.39 173.99) (width 1) (layer B.Cu) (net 13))
 (segment (start 67.31 173.99) (end 67.31 175.26) (width 1) (layer B.Cu) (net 14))
 (segment (start 67.31 175.26) (end 68.58 176.53) (width 1) (layer B.Cu) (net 14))
 (segment (start 68.58 176.53) (end 76.2 176.53) (width 1) (layer B.Cu) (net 14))
 (segment (start 77.47 175.26) (end 77.47 171.45) (width 1) (layer B.Cu) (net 14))
 (segment (start 76.2 176.53) (end 77.47 175.26) (width 1) (layer B.Cu) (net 14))
 (segment (start 73.025 161.29) (end 73.025 158.75) (width 1) (layer B.Cu) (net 9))
 (segment (start 62.23 172.085) (end 73.025 161.29) (width 1) (layer B.Cu) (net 9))
 (segment (start 62.23 173.99) (end 62.23 172.085) (width 1) (layer B.Cu) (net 9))
 (segment (start 59.69 173.99) (end 59.69 162.56) (width 1) (layer B.Cu) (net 10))
 (segment (start 59.69 162.56) (end 66.675 155.575) (width 1) (layer B.Cu) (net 10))
 (segment (start 66.675 155.575) (end 71.755 155.575) (width 1) (layer B.Cu) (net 10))
 (segment (start 73.025 154.305) (end 73.025 152.4) (width 1) (layer B.Cu) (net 10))
 (segment (start 71.755 155.575) (end 73.025 154.305) (width 1) (layer B.Cu) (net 10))
 (segment (start 82.55 159.385) (end 89.535 152.4) (width 1) (layer B.Cu) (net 11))
 (segment (start 82.55 171.45) (end 82.55 159.385) (width 1) (layer B.Cu) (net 11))
 (segment (start 57.15 173.99) (end 57.15 177.165) (width 1) (layer B.Cu) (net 11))
 (segment (start 57.15 177.165) (end 58.42 178.435) (width 1) (layer B.Cu) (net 11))
 (segment (start 58.42 178.435) (end 81.28 178.435) (width 1) (layer B.Cu) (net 11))
 (segment (start 82.55 177.165) (end 82.55 171.45) (width 1) (layer B.Cu) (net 11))
 (segment (start 81.28 178.435) (end 82.55 177.165) (width 1) (layer B.Cu) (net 11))
 (segment (start 52.07 159.385) (end 52.705 158.75) (width 1) (layer B.Cu) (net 6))
 (segment (start 52.07 173.99) (end 52.07 159.385) (width 1) (layer B.Cu) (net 6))
 (segment (start 52.705 158.75) (end 59.055 152.4) (width 1) (layer B.Cu) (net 6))
 (segment (start 59.055 152.4) (end 69.215 152.4) (width 1) (layer B.Cu) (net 6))
 (segment (start 52.705 152.4) (end 52.705 154.305) (width 1) (layer B.Cu) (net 7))
 (segment (start 52.705 154.305) (end 51.435 155.575) (width 1) (layer B.Cu) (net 7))
 (segment (start 51.435 155.575) (end 46.99 155.575) (width 1) (layer B.Cu) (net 7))
 (segment (start 46.99 155.575) (end 45.72 156.845) (width 1) (layer B.Cu) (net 7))
 (segment (start 45.72 156.845) (end 45.72 160.655) (width 1) (layer B.Cu) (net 7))
 (segment (start 49.53 164.465) (end 49.53 173.99) (width 1) (layer B.Cu) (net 7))
 (segment (start 45.72 160.655) (end 49.53 164.465) (width 1) (layer B.Cu) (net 7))
 (segment (start 32.385 158.75) (end 32.385 173.99) (width 1) (layer B.Cu) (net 2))
 (segment (start 32.385 173.99) (end 34.925 176.53) (width 1) (layer B.Cu) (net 2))
 (segment (start 34.925 176.53) (end 44.45 176.53) (width 1) (layer B.Cu) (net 2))
 (segment (start 44.45 176.53) (end 46.99 173.99) (width 1) (layer B.Cu) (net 2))
 (segment (start 85.09 163.195) (end 89.535 158.75) (width 1) (layer B.Cu) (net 12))
 (segment (start 85.09 171.45) (end 85.09 163.195) (width 1) (layer B.Cu) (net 12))
 (segment (start 48.895 146.05) (end 52.705 146.05) (width 1) (layer B.Cu) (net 1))
 (segment (start 52.705 146.05) (end 69.215 146.05) (width 1) (layer B.Cu) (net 1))
 (segment (start 69.215 146.05) (end 73.025 146.05) (width 1) (layer B.Cu) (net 1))
 (segment (start 45.72 146.05) (end 48.895 146.05) (width 1) (layer B.Cu) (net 1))
 (segment (start 45.72 168.91) (end 45.72 164.465) (width 1) (layer B.Cu) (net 1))
 (segment (start 32.385 146.05) (end 42.545 146.05) (width 1) (layer B.Cu) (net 1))
 (segment (start 42.545 146.05) (end 45.72 146.05) (width 1) (layer B.Cu) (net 1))
 (segment (start 45.72 164.465) (end 42.545 161.29) (width 1) (layer B.Cu) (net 1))
 (segment (start 42.545 161.29) (end 42.545 146.05) (width 1) (layer B.Cu) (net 1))
 (segment (start 80.01 146.05) (end 89.535 146.05) (width 1) (layer B.Cu) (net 1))
 (segment (start 73.025 146.05) (end 80.01 146.05) (width 1) (layer B.Cu) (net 1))
 (segment (start 87.63 171.45) (end 88.9 170.18) (width 1) (layer B.Cu) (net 1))
 (segment (start 88.9 170.18) (end 88.9 166.37) (width 1) (layer B.Cu) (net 1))
 (via (at 88.265 166.37) (size 1.6) (drill 0.8) (layers F.Cu B.Cu) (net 1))
 (via (at 79.375 166.37) (size 1.6) (drill 0.8) (layers F.Cu B.Cu) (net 1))
 (segment (start 78.74 166.37) (end 80.01 166.37) (width 1) (layer B.Cu) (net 1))
 (segment (start 80.01 166.37) (end 80.01 146.05) (width 1) (layer B.Cu) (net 1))
 (segment (start 80.01 171.45) (end 80.01 166.37) (width 1) (layer B.Cu) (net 1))
 (segment (start 88.265 166.37) (end 79.375 166.37) (width 1) (layer F.Cu) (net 1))
 (segment (start 35.56 155.575) (end 35.56 168.91) (width 1) (layer B.Cu) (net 3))
 (segment (start 32.385 152.4) (end 35.56 155.575) (width 1) (layer B.Cu) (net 3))
 (segment (start 35.56 168.91) (end 35.56 173.355) (width 1) (layer B.Cu) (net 3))
 (segment (start 36.195 173.99) (end 42.545 173.99) (width 1) (layer B.Cu) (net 3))
 (segment (start 35.56 173.355) (end 36.195 173.99) (width 1) (layer B.Cu) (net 3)))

